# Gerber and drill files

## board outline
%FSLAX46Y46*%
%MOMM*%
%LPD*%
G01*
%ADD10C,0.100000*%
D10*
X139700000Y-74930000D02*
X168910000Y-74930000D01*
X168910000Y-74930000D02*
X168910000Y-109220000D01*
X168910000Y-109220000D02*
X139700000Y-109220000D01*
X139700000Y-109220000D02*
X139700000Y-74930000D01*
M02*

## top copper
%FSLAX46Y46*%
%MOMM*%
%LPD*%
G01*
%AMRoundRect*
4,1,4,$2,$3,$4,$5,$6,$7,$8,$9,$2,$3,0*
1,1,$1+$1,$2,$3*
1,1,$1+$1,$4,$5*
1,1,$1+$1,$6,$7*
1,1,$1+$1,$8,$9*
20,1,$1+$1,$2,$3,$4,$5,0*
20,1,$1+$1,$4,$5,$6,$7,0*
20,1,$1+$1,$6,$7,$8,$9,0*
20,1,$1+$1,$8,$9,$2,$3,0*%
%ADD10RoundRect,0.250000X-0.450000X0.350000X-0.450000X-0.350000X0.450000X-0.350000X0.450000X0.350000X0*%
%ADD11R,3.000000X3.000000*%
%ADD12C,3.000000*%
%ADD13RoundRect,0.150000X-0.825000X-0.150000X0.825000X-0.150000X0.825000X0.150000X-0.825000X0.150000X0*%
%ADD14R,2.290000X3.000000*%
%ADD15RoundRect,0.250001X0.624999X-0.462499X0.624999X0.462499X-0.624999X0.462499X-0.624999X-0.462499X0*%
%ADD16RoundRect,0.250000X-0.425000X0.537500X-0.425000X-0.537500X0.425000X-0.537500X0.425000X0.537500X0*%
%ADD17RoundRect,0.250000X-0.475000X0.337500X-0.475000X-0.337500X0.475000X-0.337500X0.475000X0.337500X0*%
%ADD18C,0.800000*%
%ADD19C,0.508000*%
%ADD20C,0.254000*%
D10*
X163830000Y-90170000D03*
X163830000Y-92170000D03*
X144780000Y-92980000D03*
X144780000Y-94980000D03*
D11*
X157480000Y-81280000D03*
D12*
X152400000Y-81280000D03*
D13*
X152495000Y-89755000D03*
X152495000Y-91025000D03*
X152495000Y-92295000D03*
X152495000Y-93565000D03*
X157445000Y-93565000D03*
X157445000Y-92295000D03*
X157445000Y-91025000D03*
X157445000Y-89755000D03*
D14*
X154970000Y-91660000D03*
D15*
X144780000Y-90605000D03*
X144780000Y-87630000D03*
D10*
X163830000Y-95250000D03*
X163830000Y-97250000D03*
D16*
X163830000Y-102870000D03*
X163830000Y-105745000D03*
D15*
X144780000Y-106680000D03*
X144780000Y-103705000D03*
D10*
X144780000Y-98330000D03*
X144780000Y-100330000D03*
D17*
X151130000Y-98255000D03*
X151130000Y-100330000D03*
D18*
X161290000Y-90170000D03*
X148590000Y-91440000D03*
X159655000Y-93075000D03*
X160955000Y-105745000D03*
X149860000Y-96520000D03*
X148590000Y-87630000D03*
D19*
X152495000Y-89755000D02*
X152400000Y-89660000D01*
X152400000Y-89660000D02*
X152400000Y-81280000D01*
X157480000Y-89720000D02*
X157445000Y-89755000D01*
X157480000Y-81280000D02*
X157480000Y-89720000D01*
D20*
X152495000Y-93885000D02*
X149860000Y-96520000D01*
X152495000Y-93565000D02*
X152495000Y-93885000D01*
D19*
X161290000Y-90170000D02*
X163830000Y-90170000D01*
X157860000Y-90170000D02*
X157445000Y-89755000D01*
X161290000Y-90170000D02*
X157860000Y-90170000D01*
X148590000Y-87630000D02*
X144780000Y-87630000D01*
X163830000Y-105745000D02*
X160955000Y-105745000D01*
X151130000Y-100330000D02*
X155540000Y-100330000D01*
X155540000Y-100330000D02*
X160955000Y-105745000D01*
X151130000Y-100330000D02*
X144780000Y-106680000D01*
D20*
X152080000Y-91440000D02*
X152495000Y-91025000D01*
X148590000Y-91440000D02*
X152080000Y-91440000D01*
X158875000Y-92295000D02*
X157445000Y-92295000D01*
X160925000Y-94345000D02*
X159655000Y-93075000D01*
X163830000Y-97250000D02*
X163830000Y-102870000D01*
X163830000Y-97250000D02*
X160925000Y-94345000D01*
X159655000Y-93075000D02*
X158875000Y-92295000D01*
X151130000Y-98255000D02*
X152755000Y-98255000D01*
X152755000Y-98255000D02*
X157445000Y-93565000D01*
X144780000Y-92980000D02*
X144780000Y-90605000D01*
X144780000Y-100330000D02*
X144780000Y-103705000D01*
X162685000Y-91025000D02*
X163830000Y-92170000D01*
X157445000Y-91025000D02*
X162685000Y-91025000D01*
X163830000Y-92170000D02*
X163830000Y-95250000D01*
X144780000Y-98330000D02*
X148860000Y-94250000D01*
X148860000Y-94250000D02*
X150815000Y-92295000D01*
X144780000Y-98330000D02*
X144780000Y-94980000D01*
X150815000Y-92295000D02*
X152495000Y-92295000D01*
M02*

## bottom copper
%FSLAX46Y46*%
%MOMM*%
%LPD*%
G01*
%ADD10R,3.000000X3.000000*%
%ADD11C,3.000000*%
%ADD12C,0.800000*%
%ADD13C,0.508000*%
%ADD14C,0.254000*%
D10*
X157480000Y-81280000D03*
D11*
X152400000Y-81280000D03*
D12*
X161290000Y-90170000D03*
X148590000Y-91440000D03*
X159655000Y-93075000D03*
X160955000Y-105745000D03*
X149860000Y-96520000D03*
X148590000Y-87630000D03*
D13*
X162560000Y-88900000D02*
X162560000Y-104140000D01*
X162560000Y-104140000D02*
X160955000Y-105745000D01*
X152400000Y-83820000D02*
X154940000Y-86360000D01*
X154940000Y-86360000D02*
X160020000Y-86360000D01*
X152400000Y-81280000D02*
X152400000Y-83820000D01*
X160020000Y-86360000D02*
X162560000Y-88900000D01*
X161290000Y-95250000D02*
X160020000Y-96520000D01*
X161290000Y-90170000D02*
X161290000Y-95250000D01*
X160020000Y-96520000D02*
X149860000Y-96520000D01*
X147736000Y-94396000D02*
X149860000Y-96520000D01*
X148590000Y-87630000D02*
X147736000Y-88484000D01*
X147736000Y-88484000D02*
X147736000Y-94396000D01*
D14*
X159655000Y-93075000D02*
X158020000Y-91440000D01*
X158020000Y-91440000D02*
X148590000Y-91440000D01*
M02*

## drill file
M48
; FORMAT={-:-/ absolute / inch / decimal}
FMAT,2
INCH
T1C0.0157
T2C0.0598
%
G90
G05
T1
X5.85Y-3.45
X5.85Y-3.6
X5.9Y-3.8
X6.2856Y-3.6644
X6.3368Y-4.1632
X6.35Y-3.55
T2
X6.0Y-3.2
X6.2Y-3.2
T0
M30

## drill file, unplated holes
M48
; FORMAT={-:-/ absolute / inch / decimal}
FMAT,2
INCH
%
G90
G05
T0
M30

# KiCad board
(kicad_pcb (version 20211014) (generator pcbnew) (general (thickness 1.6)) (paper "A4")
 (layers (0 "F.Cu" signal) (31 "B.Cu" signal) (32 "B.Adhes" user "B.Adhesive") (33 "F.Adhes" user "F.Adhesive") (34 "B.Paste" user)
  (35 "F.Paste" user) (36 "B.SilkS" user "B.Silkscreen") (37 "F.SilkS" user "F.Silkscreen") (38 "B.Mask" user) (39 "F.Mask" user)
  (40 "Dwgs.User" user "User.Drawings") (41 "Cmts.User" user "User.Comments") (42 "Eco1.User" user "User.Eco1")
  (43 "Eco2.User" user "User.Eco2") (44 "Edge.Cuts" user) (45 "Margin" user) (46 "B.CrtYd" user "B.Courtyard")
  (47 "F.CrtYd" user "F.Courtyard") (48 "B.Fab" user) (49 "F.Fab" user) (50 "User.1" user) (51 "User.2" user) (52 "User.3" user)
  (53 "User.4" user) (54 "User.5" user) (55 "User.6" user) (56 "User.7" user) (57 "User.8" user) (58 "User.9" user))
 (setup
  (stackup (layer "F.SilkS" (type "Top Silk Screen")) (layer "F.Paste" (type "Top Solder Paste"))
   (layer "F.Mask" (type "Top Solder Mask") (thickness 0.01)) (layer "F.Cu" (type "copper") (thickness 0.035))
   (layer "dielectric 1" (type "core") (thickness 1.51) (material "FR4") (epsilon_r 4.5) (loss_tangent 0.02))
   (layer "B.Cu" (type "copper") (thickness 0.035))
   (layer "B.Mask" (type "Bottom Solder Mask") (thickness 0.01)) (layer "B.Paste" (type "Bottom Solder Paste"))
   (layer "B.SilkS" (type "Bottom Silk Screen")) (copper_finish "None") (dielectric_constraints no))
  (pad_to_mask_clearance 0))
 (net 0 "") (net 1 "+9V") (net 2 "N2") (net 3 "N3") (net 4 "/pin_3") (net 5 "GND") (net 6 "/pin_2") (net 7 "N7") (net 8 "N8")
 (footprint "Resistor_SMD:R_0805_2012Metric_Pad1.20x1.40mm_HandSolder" (layer "F.Cu") (at 163.83 91.17 -90)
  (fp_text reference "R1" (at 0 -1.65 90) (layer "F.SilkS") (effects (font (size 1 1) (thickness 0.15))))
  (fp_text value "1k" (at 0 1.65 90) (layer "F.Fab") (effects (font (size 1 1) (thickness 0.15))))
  (pad "1" smd roundrect (at -1 0 270) (size 1.2 1.4) (layers "F.Cu" "F.Paste" "F.Mask") (roundrect_rratio 0.2083333333) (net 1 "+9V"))
  (pad "2" smd roundrect (at 1 0 270) (size 1.2 1.4) (layers "F.Cu" "F.Paste" "F.Mask") (roundrect_rratio 0.2083333333) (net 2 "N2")))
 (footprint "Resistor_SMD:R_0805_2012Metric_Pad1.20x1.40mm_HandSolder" (layer "F.Cu") (at 144.78 93.98 -90)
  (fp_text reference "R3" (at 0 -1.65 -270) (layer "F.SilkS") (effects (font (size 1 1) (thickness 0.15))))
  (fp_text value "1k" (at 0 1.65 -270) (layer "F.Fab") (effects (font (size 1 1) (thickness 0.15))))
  (pad "1" smd roundrect (at -1 0 270) (size 1.2 1.4) (layers "F.Cu" "F.Paste" "F.Mask") (roundrect_rratio 0.2083333333) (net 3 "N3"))
  (pad "2" smd roundrect (at 1 0 270) (size 1.2 1.4) (layers "F.Cu" "F.Paste" "F.Mask") (roundrect_rratio 0.2083333333) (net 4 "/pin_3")))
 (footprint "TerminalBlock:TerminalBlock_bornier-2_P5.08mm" (layer "F.Cu") (at 157.48 81.28 180)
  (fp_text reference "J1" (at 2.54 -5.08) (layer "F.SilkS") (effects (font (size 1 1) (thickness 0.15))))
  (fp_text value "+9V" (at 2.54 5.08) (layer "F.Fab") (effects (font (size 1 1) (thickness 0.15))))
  (pad "1" thru_hole rect (at 0 0 180) (size 3 3) (drill 1.52) (layers *.Cu *.Mask) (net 1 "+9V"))
  (pad "2" thru_hole circle (at 5.08 0 180) (size 3 3) (drill 1.52) (layers *.Cu *.Mask) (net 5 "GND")))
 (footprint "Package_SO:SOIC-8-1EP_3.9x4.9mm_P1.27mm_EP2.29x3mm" (layer "F.Cu") (at 154.97 91.66)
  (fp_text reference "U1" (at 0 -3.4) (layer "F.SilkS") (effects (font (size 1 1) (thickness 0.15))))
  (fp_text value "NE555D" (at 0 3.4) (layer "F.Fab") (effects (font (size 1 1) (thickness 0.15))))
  (pad "" smd roundrect (at 0.57 -0.75) (size 0.92 1.21) (layers "F.Paste") (roundrect_rratio 0.25))
  (pad "" smd roundrect (at 0.57 0.75) (size 0.92 1.21) (layers "F.Paste") (roundrect_rratio 0.25))
  (pad "" smd roundrect (at -0.57 -0.75) (size 0.92 1.21) (layers "F.Paste") (roundrect_rratio 0.25))
  (pad "" smd roundrect (at -0.57 0.75) (size 0.92 1.21) (layers "F.Paste") (roundrect_rratio 0.25))
  (pad "1" smd roundrect (at -2.475 -1.905) (size 1.95 0.6) (layers "F.Cu" "F.Paste" "F.Mask") (roundrect_rratio 0.25) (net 5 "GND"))
  (pad "2" smd roundrect (at -2.475 -0.635) (size 1.95 0.6) (layers "F.Cu" "F.Paste" "F.Mask") (roundrect_rratio 0.25) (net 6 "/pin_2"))
  (pad "3" smd roundrect (at -2.475 0.635) (size 1.95 0.6) (layers "F.Cu" "F.Paste" "F.Mask") (roundrect_rratio 0.25) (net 4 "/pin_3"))
  (pad "4" smd roundrect (at -2.475 1.905) (size 1.95 0.6) (layers "F.Cu" "F.Paste" "F.Mask") (roundrect_rratio 0.25) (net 1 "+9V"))
  (pad "5" smd roundrect (at 2.475 1.905) (size 1.95 0.6) (layers "F.Cu" "F.Paste" "F.Mask") (roundrect_rratio 0.25) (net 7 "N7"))
  (pad "6" smd roundrect (at 2.475 0.635) (size 1.95 0.6) (layers "F.Cu" "F.Paste" "F.Mask") (roundrect_rratio 0.25) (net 6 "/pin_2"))
  (pad "7" smd roundrect (at 2.475 -0.635) (size 1.95 0.6) (layers "F.Cu" "F.Paste" "F.Mask") (roundrect_rratio 0.25) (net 2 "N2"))
  (pad "8" smd roundrect (at 2.475 -1.905) (size 1.95 0.6) (layers "F.Cu" "F.Paste" "F.Mask") (roundrect_rratio 0.25) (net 1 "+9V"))
  (pad "9" smd rect (at 0 0) (size 2.29 3) (layers "F.Cu" "F.Mask")))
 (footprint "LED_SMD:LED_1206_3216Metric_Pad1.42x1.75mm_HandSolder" (layer "F.Cu") (at 144.78 89.1175 90)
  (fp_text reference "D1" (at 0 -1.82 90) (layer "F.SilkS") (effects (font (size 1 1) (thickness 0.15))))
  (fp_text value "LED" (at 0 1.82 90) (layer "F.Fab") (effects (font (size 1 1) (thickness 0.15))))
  (pad "1" smd roundrect (at -1.4875 0 90) (size 1.425 1.75) (layers "F.Cu" "F.Paste" "F.Mask") (roundrect_rratio 0.1754392982) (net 3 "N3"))
  (pad "2" smd roundrect (at 1.4875 0 90) (size 1.425 1.75) (layers "F.Cu" "F.Paste" "F.Mask") (roundrect_rratio 0.1754392982) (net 1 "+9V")))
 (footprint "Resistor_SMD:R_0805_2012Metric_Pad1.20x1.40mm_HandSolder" (layer "F.Cu") (at 163.83 96.25 -90)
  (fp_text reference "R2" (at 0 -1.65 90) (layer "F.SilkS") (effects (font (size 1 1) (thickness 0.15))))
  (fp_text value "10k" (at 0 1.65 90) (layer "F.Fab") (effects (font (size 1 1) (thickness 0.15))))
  (pad "1" smd roundrect (at -1 0 270) (size 1.2 1.4) (layers "F.Cu" "F.Paste" "F.Mask") (roundrect_rratio 0.2083333333) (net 2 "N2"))
  (pad "2" smd roundrect (at 1 0 270) (size 1.2 1.4) (layers "F.Cu" "F.Paste" "F.Mask") (roundrect_rratio 0.2083333333) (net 6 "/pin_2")))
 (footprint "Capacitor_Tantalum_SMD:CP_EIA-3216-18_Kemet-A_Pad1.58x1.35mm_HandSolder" (layer "F.Cu") (at 163.83 104.3075 -90)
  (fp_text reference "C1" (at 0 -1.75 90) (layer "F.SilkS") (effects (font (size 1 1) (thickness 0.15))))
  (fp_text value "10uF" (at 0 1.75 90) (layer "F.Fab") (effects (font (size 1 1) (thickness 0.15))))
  (pad "1" smd roundrect (at -1.4375 0 270) (size 1.575 1.35) (layers "F.Cu" "F.Paste" "F.Mask") (roundrect_rratio 0.1851851852)
   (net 6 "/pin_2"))
  (pad "2" smd roundrect (at 1.4375 0 270) (size 1.575 1.35) (layers "F.Cu" "F.Paste" "F.Mask") (roundrect_rratio 0.1851851852)
   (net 5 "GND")))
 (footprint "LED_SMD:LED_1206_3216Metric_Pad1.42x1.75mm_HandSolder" (layer "F.Cu") (at 144.78 105.1925 90)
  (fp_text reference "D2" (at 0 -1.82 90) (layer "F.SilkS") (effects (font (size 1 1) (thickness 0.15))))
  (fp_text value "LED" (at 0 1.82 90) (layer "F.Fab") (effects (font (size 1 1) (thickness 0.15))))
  (pad "1" smd roundrect (at -1.4875 0 90) (size 1.425 1.75) (layers "F.Cu" "F.Paste" "F.Mask") (roundrect_rratio 0.1754392982)
   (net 5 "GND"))
  (pad "2" smd roundrect (at 1.4875 0 90) (size 1.425 1.75) (layers "F.Cu" "F.Paste" "F.Mask") (roundrect_rratio 0.1754392982) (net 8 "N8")))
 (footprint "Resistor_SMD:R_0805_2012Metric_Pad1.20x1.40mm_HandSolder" (layer "F.Cu") (at 144.78 99.33 -90)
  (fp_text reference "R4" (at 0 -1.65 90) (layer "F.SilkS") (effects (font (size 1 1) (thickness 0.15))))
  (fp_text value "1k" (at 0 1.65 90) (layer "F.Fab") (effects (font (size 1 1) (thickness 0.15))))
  (pad "1" smd roundrect (at -1 0 270) (size 1.2 1.4) (layers "F.Cu" "F.Paste" "F.Mask") (roundrect_rratio 0.2083333333) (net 4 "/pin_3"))
  (pad "2" smd roundrect (at 1 0 270) (size 1.2 1.4) (layers "F.Cu" "F.Paste" "F.Mask") (roundrect_rratio 0.2083333333) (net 8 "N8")))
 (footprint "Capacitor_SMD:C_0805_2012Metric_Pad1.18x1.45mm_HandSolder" (layer "F.Cu") (at 151.13 99.2925 -90)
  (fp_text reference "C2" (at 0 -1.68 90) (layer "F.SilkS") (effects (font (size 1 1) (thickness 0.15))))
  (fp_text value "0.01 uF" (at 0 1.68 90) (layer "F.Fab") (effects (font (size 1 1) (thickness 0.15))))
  (pad "1" smd roundrect (at -1.0375 0 270) (size 1.175 1.45) (layers "F.Cu" "F.Paste" "F.Mask") (roundrect_rratio 0.2127659574)
   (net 7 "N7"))
  (pad "2" smd roundrect (at 1.0375 0 270) (size 1.175 1.45) (layers "F.Cu" "F.Paste" "F.Mask") (roundrect_rratio 0.2127659574)
   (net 5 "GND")))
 (gr_rect (start 139.7 74.93) (end 168.91 109.22) (layer "Edge.Cuts") (width 0.1) (fill none))
 (segment (start 152.08 91.44) (end 152.495 91.025) (width 0.254) (layer "F.Cu") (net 6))
 (segment (start 148.59 91.44) (end 152.08 91.44) (width 0.254) (layer "F.Cu") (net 6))
 (segment (start 158.875 92.295) (end 157.445 92.295) (width 0.254) (layer "F.Cu") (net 6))
 (segment (start 160.925 94.345) (end 159.655 93.075) (width 0.254) (layer "F.Cu") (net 6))
 (segment (start 163.83 97.25) (end 163.83 102.87) (width 0.254) (layer "F.Cu") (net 6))
 (segment (start 163.83 97.25) (end 160.925 94.345) (width 0.254) (layer "F.Cu") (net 6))
 (segment (start 159.655 93.075) (end 158.875 92.295) (width 0.254) (layer "F.Cu") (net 6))
 (via (at 148.59 91.44) (size 0.8) (drill 0.4) (layers "F.Cu" "B.Cu") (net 6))
 (via (at 159.655 93.075) (size 0.8) (drill 0.4) (layers "F.Cu" "B.Cu") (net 6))
 (segment (start 159.655 93.075) (end 158.02 91.44) (width 0.254) (layer "B.Cu") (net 6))
 (segment (start 158.02 91.44) (end 148.59 91.44) (width 0.254) (layer "B.Cu") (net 6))
 (segment (start 151.13 100.33) (end 155.54 100.33) (width 0.508) (layer "F.Cu") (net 5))
 (segment (start 151.13 100.33) (end 144.78 106.68) (width 0.508) (layer "F.Cu") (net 5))
 (segment (start 155.54 100.33) (end 160.955 105.745) (width 0.508) (layer "F.Cu") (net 5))
 (segment (start 152.4 89.66) (end 152.4 81.28) (width 0.508) (layer "F.Cu") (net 5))
 (segment (start 152.495 89.755) (end 152.4 89.66) (width 0.508) (layer "F.Cu") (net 5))
 (segment (start 163.83 105.745) (end 160.955 105.745) (width 0.508) (layer "F.Cu") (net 5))
 (via (at 160.955 105.745) (size 0.8) (drill 0.4) (layers "F.Cu" "B.Cu") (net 5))
 (segment (start 162.56 104.14) (end 160.955 105.745) (width 0.508) (layer "B.Cu") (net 5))
 (segment (start 152.4 81.28) (end 152.4 83.82) (width 0.508) (layer "B.Cu") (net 5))
 (segment (start 152.4 83.82) (end 154.94 86.36) (width 0.508) (layer "B.Cu") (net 5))
 (segment (start 154.94 86.36) (end 160.02 86.36) (width 0.508) (layer "B.Cu") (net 5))
 (segment (start 160.02 86.36) (end 162.56 88.9) (width 0.508) (layer "B.Cu") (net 5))
 (segment (start 162.56 88.9) (end 162.56 104.14) (width 0.508) (layer "B.Cu") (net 5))
 (segment (start 151.13 98.255) (end 152.755 98.255) (width 0.254) (layer "F.Cu") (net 7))
 (segment (start 152.755 98.255) (end 157.445 93.565) (width 0.254) (layer "F.Cu") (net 7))
 (segment (start 144.78 92.98) (end 144.78 90.605) (width 0.254) (layer "F.Cu") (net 3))
 (segment (start 161.29 90.17) (end 157.86 90.17) (width 0.508) (layer "F.Cu") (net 1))
 (segment (start 152.495 93.565) (end 152.495 93.885) (width 0.254) (layer "F.Cu") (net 1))
 (segment (start 148.59 87.63) (end 144.78 87.63) (width 0.508) (layer "F.Cu") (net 1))
 (segment (start 161.29 90.17) (end 163.83 90.17) (width 0.508) (layer "F.Cu") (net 1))
 (segment (start 157.48 81.28) (end 157.48 89.72) (width 0.508) (layer "F.Cu") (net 1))
 (segment (start 157.48 89.72) (end 157.445 89.755) (width 0.508) (layer "F.Cu") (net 1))
 (segment (start 157.86 90.17) (end 157.445 89.755) (width 0.508) (layer "F.Cu") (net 1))
 (segment (start 152.495 93.885) (end 149.86 96.52) (width 0.254) (layer "F.Cu") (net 1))
 (via (at 161.29 90.17) (size 0.8) (drill 0.4) (layers "F.Cu" "B.Cu") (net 1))
 (via (at 149.86 96.52) (size 0.8) (drill 0.4) (layers "F.Cu" "B.Cu") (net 1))
 (via (at 148.59 87.63) (size 0.8) (drill 0.4) (layers "F.Cu" "B.Cu") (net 1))
 (segment (start 148.59 87.63) (end 147.736 88.484) (width 0.508) (layer "B.Cu") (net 1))
 (segment (start 147.736 88.484) (end 147.736 94.396) (width 0.508) (layer "B.Cu") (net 1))
 (segment (start 147.736 94.396) (end 149.86 96.52) (width 0.508) (layer "B.Cu") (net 1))
 (segment (start 161.29 90.17) (end 161.29 95.25) (width 0.508) (layer "B.Cu") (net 1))
 (segment (start 160.02 96.52) (end 149.86 96.52) (width 0.508) (layer "B.Cu") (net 1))
 (segment (start 161.29 95.25) (end 160.02 96.52) (width 0.508) (layer "B.Cu") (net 1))
 (segment (start 144.78 100.33) (end 144.78 103.705) (width 0.254) (layer "F.Cu") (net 8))
 (segment (start 162.685 91.025) (end 163.83 92.17) (width 0.254) (layer "F.Cu") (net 2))
 (segment (start 157.445 91.025) (end 162.685 91.025) (width 0.254) (layer "F.Cu") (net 2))
 (segment (start 163.83 92.17) (end 163.83 95.25) (width 0.254) (layer "F.Cu") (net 2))
 (segment (start 144.78 98.33) (end 148.86 94.25) (width 0.254) (layer "F.Cu") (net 4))
 (segment (start 148.86 94.25) (end 150.815 92.295) (width 0.254) (layer "F.Cu") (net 4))
 (segment (start 144.78 98.33) (end 144.78 94.98) (width 0.254) (layer "F.Cu") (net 4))
 (segment (start 150.815 92.295) (end 152.495 92.295) (width 0.254) (layer "F.Cu") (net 4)))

